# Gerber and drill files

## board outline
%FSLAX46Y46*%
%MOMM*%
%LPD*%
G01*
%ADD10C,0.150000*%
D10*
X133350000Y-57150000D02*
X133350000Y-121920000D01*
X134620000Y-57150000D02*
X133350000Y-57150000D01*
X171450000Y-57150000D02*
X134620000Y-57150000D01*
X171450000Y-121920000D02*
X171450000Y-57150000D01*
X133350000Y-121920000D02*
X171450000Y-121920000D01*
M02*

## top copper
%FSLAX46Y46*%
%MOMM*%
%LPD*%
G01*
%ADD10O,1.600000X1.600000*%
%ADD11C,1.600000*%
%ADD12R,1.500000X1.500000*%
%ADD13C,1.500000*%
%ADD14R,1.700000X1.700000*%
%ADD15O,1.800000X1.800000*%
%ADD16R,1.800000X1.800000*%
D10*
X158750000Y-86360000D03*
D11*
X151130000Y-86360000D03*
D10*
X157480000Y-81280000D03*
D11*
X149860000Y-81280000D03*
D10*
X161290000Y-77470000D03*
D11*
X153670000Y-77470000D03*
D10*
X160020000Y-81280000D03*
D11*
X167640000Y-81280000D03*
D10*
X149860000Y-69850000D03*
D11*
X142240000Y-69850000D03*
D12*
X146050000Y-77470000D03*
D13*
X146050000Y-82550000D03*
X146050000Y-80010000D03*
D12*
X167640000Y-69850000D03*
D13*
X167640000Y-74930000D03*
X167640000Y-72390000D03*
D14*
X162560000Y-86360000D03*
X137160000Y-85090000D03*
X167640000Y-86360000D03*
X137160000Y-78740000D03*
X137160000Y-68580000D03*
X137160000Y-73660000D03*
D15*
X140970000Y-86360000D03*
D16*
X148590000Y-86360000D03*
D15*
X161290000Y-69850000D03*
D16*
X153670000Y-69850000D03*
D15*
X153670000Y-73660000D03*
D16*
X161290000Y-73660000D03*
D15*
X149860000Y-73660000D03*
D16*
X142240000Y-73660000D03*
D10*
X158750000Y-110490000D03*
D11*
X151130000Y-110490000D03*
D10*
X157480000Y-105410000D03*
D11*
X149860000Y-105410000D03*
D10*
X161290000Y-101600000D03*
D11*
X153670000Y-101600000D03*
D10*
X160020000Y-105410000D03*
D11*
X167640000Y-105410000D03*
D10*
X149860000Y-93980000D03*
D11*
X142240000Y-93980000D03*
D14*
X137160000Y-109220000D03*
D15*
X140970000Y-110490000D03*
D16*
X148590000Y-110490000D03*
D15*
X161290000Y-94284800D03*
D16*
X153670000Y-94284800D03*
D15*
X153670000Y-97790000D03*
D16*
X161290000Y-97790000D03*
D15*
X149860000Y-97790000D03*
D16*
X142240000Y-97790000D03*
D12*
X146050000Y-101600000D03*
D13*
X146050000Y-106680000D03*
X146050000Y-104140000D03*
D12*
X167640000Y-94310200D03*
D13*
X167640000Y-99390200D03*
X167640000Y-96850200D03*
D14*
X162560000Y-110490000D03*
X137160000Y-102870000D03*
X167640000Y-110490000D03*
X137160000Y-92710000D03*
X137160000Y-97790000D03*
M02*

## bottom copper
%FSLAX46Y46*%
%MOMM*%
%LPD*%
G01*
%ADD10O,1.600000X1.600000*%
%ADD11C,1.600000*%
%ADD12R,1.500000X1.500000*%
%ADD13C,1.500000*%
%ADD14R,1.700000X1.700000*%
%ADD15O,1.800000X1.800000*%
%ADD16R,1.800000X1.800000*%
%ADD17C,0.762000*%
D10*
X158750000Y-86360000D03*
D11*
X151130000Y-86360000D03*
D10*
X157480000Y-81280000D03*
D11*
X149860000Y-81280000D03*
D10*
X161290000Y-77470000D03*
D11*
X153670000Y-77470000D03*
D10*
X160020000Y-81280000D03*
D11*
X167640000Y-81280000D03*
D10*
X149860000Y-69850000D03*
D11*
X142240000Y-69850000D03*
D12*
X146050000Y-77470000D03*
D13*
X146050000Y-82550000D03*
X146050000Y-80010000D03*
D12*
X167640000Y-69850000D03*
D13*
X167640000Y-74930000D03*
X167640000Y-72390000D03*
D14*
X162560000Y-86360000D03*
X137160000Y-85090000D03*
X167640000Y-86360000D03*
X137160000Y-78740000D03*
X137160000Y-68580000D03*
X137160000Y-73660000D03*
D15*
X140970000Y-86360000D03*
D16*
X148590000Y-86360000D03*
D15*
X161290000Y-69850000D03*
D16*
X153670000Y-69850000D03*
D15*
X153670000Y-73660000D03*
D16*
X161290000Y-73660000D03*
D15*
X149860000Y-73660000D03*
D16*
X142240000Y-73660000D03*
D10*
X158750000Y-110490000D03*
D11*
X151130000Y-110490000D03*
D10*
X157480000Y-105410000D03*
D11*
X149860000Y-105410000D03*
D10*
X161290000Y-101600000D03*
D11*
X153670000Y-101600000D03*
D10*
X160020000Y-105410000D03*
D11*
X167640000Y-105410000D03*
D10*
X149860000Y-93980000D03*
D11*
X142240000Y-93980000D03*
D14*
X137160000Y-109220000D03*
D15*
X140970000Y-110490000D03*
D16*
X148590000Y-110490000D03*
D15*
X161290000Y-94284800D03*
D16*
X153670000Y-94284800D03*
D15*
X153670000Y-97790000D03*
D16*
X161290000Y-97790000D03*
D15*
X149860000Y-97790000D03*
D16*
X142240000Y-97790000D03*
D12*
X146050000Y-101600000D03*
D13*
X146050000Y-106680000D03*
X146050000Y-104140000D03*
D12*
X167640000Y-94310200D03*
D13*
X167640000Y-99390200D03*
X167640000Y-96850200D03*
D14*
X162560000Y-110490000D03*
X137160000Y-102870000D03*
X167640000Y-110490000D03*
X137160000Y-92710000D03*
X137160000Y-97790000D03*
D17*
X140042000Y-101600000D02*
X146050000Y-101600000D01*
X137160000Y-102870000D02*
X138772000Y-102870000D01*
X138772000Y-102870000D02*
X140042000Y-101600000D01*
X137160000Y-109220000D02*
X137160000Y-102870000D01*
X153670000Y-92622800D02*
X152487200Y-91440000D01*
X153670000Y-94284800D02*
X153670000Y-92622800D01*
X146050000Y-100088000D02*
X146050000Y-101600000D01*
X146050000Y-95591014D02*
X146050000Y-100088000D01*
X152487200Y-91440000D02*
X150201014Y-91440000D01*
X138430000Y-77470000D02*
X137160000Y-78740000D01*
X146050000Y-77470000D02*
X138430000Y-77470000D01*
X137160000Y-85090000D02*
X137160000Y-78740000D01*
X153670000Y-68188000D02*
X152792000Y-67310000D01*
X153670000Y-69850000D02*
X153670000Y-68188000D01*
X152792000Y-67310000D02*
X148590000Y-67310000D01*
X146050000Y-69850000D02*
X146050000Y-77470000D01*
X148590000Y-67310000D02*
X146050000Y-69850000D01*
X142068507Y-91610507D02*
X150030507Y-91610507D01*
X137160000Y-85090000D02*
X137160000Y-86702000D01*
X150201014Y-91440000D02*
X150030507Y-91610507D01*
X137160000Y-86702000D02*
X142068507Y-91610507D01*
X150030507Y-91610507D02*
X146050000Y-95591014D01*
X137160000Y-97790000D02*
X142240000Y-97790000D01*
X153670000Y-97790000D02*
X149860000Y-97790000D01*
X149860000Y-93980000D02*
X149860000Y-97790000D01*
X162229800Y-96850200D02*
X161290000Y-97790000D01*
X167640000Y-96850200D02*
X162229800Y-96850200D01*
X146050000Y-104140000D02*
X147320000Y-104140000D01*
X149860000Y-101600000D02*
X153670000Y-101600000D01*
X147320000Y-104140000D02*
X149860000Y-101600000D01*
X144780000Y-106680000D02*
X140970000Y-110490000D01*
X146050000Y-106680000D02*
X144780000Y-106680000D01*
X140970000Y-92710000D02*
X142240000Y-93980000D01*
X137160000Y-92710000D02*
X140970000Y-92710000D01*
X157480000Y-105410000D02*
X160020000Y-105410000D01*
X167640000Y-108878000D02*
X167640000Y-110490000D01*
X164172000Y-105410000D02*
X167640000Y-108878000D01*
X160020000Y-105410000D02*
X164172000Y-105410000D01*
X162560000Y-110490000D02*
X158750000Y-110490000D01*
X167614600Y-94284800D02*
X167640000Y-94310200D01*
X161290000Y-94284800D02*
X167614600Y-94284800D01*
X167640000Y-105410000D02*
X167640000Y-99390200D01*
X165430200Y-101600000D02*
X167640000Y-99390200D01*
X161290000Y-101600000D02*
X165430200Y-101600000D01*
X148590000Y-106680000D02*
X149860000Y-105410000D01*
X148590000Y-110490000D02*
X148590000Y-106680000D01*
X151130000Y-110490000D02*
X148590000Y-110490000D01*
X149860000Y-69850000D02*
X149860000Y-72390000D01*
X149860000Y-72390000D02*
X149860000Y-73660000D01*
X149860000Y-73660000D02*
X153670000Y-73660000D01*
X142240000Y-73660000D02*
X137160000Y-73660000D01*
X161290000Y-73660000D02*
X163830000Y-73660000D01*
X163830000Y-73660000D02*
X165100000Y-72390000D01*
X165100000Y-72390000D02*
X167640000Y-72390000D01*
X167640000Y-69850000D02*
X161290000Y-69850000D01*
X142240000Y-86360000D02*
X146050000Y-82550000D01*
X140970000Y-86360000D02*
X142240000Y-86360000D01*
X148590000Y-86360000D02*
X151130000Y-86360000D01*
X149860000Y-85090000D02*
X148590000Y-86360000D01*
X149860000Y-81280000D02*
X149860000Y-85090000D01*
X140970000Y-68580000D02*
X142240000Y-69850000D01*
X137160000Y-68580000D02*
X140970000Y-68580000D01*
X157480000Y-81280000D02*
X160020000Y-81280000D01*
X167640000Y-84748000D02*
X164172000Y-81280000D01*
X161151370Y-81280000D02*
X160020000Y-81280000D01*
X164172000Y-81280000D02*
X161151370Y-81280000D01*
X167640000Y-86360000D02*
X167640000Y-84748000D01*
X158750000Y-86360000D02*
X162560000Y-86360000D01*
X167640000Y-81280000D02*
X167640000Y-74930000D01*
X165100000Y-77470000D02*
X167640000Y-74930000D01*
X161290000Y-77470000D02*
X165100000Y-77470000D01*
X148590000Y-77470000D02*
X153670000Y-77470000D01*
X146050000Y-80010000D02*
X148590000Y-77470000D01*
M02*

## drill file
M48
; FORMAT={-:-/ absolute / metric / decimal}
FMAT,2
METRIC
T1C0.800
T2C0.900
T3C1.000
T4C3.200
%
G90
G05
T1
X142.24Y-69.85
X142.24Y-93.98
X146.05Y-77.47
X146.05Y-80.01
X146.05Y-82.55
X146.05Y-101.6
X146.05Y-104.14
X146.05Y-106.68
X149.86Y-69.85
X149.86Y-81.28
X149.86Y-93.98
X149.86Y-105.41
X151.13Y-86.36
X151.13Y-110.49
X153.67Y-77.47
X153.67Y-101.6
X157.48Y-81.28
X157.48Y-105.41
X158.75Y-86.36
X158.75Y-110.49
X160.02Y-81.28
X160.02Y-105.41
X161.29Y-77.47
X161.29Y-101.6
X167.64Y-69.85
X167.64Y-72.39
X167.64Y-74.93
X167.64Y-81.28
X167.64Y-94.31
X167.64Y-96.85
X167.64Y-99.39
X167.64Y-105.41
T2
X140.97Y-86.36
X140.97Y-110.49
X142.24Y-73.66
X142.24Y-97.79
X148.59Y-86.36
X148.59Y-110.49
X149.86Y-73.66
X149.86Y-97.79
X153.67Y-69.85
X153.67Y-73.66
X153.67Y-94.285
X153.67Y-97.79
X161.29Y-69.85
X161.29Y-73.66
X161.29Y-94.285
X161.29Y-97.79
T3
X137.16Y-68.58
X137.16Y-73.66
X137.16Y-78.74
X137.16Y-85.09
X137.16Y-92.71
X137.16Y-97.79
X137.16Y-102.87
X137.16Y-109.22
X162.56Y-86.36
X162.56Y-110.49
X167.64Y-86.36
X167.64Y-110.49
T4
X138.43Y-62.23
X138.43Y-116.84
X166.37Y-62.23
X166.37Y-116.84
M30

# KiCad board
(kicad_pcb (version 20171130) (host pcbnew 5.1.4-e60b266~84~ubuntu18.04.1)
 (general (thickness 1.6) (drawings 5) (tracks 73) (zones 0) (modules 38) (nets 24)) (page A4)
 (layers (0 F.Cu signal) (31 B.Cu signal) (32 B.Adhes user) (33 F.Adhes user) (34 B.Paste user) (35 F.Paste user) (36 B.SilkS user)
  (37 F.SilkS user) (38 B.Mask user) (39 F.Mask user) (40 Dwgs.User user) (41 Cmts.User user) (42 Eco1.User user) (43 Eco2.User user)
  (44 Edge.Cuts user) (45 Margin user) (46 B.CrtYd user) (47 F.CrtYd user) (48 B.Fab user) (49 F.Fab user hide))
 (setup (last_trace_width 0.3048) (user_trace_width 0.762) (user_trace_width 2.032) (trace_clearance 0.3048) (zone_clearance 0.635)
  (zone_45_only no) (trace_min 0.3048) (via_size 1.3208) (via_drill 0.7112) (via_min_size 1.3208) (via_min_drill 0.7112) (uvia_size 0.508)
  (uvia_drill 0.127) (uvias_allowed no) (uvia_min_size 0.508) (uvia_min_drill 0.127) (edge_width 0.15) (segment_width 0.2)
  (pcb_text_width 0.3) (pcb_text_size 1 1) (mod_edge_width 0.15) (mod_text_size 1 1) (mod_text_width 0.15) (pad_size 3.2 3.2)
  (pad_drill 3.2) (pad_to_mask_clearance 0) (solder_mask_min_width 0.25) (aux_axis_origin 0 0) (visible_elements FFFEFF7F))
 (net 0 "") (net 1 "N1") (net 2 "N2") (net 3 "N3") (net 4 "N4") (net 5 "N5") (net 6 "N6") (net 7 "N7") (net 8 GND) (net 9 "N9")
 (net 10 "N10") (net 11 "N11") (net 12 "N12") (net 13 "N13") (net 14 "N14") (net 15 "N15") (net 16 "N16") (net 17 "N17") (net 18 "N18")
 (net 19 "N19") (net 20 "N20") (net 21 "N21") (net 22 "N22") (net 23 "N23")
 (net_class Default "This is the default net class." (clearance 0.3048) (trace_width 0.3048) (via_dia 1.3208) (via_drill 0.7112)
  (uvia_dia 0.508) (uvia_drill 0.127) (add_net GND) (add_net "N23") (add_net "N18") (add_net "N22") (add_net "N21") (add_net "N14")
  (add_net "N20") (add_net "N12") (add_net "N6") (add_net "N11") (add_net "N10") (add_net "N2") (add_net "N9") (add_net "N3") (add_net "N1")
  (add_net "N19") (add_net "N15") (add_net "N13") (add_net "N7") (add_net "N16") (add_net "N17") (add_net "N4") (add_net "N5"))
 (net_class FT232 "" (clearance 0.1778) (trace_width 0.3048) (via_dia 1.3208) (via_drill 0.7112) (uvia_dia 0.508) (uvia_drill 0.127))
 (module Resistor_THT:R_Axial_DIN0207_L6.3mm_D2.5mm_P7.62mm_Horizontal (layer F.Cu) (at 151.13 86.36)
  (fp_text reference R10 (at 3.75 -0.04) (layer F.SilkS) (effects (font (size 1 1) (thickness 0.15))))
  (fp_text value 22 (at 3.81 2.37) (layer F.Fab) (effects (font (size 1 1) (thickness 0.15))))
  (pad 2 thru_hole oval (at 7.62 0) (size 1.6 1.6) (drill 0.8) (layers *.Cu *.Mask) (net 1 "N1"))
  (pad 1 thru_hole circle (at 0 0) (size 1.6 1.6) (drill 0.8) (layers *.Cu *.Mask) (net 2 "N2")))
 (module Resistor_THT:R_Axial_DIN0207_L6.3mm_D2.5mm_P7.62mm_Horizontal (layer F.Cu) (at 149.86 81.28)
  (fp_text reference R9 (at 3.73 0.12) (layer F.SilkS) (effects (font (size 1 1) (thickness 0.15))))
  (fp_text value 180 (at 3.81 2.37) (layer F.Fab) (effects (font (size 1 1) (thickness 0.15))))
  (pad 2 thru_hole oval (at 7.62 0) (size 1.6 1.6) (drill 0.8) (layers *.Cu *.Mask) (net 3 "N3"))
  (pad 1 thru_hole circle (at 0 0) (size 1.6 1.6) (drill 0.8) (layers *.Cu *.Mask) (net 2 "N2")))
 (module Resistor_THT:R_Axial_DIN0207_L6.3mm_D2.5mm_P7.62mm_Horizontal (layer F.Cu) (at 153.67 77.47)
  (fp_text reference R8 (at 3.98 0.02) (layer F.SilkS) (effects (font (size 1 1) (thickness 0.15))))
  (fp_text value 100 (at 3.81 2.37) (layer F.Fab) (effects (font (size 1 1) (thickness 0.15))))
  (pad 2 thru_hole oval (at 7.62 0) (size 1.6 1.6) (drill 0.8) (layers *.Cu *.Mask) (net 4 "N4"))
  (pad 1 thru_hole circle (at 0 0) (size 1.6 1.6) (drill 0.8) (layers *.Cu *.Mask) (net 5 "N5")))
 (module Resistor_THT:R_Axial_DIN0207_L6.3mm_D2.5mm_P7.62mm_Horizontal (layer F.Cu) (at 167.64 81.28 180)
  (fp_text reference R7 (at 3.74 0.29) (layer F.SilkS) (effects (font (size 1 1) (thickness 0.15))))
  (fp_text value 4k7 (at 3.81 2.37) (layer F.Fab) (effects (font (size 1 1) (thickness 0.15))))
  (pad 2 thru_hole oval (at 7.62 0 180) (size 1.6 1.6) (drill 0.8) (layers *.Cu *.Mask) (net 3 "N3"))
  (pad 1 thru_hole circle (at 0 0 180) (size 1.6 1.6) (drill 0.8) (layers *.Cu *.Mask) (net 4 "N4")))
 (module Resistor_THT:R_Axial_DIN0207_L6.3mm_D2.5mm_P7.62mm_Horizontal (layer F.Cu) (at 142.24 69.85)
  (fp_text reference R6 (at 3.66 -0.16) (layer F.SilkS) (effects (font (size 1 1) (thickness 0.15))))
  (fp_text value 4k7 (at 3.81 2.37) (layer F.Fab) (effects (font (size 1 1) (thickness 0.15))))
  (pad 2 thru_hole oval (at 7.62 0) (size 1.6 1.6) (drill 0.8) (layers *.Cu *.Mask) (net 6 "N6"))
  (pad 1 thru_hole circle (at 0 0) (size 1.6 1.6) (drill 0.8) (layers *.Cu *.Mask) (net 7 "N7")))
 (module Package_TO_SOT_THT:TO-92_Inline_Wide (layer F.Cu) (at 146.05 77.47 270)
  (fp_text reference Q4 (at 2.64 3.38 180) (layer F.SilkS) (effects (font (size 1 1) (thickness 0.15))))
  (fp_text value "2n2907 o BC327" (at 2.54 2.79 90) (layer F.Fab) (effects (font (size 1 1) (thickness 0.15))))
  (pad 1 thru_hole rect (at 0 0) (size 1.5 1.5) (drill 0.8) (layers *.Cu *.Mask) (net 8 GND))
  (pad 3 thru_hole circle (at 5.08 0) (size 1.5 1.5) (drill 0.8) (layers *.Cu *.Mask) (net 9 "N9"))
  (pad 2 thru_hole circle (at 2.54 0) (size 1.5 1.5) (drill 0.8) (layers *.Cu *.Mask) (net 5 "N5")))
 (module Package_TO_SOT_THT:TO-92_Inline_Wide (layer F.Cu) (at 167.64 69.85 270)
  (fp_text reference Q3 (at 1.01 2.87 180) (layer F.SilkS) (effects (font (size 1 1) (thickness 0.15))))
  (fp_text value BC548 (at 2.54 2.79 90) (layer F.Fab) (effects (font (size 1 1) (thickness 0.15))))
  (pad 1 thru_hole rect (at 0 0) (size 1.5 1.5) (drill 0.8) (layers *.Cu *.Mask) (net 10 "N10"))
  (pad 3 thru_hole circle (at 5.08 0) (size 1.5 1.5) (drill 0.8) (layers *.Cu *.Mask) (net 4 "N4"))
  (pad 2 thru_hole circle (at 2.54 0) (size 1.5 1.5) (drill 0.8) (layers *.Cu *.Mask) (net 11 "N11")))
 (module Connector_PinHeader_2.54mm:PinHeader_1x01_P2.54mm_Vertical (layer F.Cu) (at 162.56 86.36)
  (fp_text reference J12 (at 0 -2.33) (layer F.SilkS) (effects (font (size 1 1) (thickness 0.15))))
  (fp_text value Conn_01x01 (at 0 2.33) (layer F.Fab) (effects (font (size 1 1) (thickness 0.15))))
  (pad 1 thru_hole rect (at 0 0) (size 1.7 1.7) (drill 1) (layers *.Cu *.Mask) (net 1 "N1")))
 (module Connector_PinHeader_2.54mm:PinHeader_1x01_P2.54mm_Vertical (layer F.Cu) (at 137.16 85.09)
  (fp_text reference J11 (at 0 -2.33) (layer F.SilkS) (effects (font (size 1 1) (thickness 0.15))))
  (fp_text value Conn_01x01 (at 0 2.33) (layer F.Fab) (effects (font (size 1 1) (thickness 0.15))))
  (pad 1 thru_hole rect (at 0 0) (size 1.7 1.7) (drill 1) (layers *.Cu *.Mask) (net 8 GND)))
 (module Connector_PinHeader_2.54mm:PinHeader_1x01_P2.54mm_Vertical (layer F.Cu) (at 167.64 86.36)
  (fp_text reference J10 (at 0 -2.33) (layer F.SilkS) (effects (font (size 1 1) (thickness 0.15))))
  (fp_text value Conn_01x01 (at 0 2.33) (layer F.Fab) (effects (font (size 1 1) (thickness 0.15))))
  (pad 1 thru_hole rect (at 0 0) (size 1.7 1.7) (drill 1) (layers *.Cu *.Mask) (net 3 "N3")))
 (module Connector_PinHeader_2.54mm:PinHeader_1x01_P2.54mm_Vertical (layer F.Cu) (at 137.16 78.74)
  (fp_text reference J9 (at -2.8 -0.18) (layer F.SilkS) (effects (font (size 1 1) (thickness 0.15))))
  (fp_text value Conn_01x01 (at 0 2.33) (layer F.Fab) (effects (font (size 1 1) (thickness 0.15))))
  (pad 1 thru_hole rect (at 0 0) (size 1.7 1.7) (drill 1) (layers *.Cu *.Mask) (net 8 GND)))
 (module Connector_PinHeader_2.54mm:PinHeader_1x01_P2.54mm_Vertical (layer F.Cu) (at 137.16 68.58)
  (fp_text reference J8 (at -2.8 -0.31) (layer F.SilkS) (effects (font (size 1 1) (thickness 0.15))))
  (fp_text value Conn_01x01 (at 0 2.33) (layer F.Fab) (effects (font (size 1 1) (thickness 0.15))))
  (pad 1 thru_hole rect (at 0 0) (size 1.7 1.7) (drill 1) (layers *.Cu *.Mask) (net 7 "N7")))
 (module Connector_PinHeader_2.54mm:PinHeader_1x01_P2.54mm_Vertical (layer F.Cu) (at 137.16 73.66)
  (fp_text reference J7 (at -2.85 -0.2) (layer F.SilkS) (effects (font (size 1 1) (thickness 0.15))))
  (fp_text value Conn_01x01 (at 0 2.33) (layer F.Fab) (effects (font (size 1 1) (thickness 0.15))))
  (pad 1 thru_hole rect (at 0 0) (size 1.7 1.7) (drill 1) (layers *.Cu *.Mask) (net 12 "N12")))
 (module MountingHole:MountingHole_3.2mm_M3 (layer F.Cu) (at 138.43 62.23)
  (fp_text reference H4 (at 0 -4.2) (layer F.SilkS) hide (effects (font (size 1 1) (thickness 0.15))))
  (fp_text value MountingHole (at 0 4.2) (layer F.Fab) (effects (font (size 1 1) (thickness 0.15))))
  (pad 1 np_thru_hole circle (at 0 0) (size 3.2 3.2) (drill 3.2) (layers *.Cu *.Mask)))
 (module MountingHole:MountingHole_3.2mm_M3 (layer F.Cu) (at 166.37 116.84)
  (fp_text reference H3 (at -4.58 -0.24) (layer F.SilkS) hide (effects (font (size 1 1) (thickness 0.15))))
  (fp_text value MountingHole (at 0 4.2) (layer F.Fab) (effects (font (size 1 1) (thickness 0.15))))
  (pad 1 np_thru_hole circle (at 0 0) (size 3.2 3.2) (drill 3.2) (layers *.Cu *.Mask)))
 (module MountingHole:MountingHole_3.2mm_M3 (layer F.Cu) (at 138.43 116.84)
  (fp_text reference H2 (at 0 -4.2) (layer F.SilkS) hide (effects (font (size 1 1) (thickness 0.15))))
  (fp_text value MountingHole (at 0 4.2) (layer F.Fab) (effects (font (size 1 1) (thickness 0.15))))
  (pad 1 np_thru_hole circle (at 0 0) (size 3.2 3.2) (drill 3.2) (layers *.Cu *.Mask)))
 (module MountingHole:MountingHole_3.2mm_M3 (layer F.Cu) (at 166.37 62.23)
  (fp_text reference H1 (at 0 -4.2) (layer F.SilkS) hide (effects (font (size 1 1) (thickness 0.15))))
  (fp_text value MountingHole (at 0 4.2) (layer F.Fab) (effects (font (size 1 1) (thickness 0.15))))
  (pad 1 np_thru_hole circle (at 0 0) (size 3.2 3.2) (drill 3.2) (layers *.Cu *.Mask)))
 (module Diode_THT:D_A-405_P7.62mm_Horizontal (layer F.Cu) (at 148.59 86.36 180)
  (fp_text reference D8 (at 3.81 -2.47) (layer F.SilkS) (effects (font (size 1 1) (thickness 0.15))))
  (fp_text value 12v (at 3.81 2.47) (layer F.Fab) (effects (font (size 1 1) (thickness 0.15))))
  (pad 2 thru_hole oval (at 7.62 0 180) (size 1.8 1.8) (drill 0.9) (layers *.Cu *.Mask) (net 9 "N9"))
  (pad 1 thru_hole rect (at 0 0 180) (size 1.8 1.8) (drill 0.9) (layers *.Cu *.Mask) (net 2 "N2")))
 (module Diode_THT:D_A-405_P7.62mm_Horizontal (layer F.Cu) (at 153.67 69.85)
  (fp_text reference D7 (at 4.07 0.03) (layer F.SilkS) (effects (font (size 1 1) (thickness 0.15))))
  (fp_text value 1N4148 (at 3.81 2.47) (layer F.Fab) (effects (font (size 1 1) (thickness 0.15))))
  (pad 2 thru_hole oval (at 7.62 0) (size 1.8 1.8) (drill 0.9) (layers *.Cu *.Mask) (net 10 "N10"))
  (pad 1 thru_hole rect (at 0 0) (size 1.8 1.8) (drill 0.9) (layers *.Cu *.Mask) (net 8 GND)))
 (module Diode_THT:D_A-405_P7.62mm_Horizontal (layer F.Cu) (at 161.29 73.66 180)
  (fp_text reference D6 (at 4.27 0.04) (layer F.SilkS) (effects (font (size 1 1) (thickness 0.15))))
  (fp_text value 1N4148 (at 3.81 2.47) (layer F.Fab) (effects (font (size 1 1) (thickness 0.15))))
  (pad 2 thru_hole oval (at 7.62 0 180) (size 1.8 1.8) (drill 0.9) (layers *.Cu *.Mask) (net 6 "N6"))
  (pad 1 thru_hole rect (at 0 0 180) (size 1.8 1.8) (drill 0.9) (layers *.Cu *.Mask) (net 11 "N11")))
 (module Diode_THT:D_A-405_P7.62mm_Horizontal (layer F.Cu) (at 142.24 73.66)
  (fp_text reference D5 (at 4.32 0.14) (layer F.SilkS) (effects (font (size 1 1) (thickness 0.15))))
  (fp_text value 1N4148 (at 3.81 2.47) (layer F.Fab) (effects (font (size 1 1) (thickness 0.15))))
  (pad 2 thru_hole oval (at 7.62 0) (size 1.8 1.8) (drill 0.9) (layers *.Cu *.Mask) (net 6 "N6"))
  (pad 1 thru_hole rect (at 0 0) (size 1.8 1.8) (drill 0.9) (layers *.Cu *.Mask) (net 12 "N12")))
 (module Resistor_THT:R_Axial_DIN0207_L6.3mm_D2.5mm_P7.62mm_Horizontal (layer F.Cu) (at 151.13 110.49)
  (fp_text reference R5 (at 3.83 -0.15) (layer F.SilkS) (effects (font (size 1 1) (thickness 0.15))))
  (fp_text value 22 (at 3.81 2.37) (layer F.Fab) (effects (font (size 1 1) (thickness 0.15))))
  (pad 2 thru_hole oval (at 7.62 0) (size 1.6 1.6) (drill 0.8) (layers *.Cu *.Mask) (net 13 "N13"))
  (pad 1 thru_hole circle (at 0 0) (size 1.6 1.6) (drill 0.8) (layers *.Cu *.Mask) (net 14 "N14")))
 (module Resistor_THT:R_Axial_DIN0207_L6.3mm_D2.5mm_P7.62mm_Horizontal (layer F.Cu) (at 149.86 105.41)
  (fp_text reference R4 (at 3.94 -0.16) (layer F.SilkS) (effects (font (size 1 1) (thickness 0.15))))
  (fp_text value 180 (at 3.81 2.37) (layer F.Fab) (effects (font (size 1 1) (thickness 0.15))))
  (pad 2 thru_hole oval (at 7.62 0) (size 1.6 1.6) (drill 0.8) (layers *.Cu *.Mask) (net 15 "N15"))
  (pad 1 thru_hole circle (at 0 0) (size 1.6 1.6) (drill 0.8) (layers *.Cu *.Mask) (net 14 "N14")))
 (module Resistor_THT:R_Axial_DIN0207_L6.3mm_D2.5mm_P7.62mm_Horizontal (layer F.Cu) (at 153.67 101.6)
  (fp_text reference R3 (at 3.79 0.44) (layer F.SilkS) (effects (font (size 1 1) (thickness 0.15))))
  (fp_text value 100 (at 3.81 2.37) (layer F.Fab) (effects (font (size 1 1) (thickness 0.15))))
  (pad 2 thru_hole oval (at 7.62 0) (size 1.6 1.6) (drill 0.8) (layers *.Cu *.Mask) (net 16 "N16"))
  (pad 1 thru_hole circle (at 0 0) (size 1.6 1.6) (drill 0.8) (layers *.Cu *.Mask) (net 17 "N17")))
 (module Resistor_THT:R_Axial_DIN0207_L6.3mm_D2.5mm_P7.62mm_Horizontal (layer F.Cu) (at 167.64 105.41 180)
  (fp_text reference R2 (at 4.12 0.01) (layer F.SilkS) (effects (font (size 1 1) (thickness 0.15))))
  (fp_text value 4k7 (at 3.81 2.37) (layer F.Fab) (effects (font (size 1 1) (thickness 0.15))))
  (pad 2 thru_hole oval (at 7.62 0 180) (size 1.6 1.6) (drill 0.8) (layers *.Cu *.Mask) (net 15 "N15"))
  (pad 1 thru_hole circle (at 0 0 180) (size 1.6 1.6) (drill 0.8) (layers *.Cu *.Mask) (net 16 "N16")))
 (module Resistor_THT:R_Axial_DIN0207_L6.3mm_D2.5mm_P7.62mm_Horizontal (layer F.Cu) (at 142.24 93.98)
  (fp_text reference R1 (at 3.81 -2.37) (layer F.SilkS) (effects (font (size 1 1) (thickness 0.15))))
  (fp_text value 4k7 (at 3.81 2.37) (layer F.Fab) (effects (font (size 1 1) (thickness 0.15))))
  (pad 2 thru_hole oval (at 7.62 0) (size 1.6 1.6) (drill 0.8) (layers *.Cu *.Mask) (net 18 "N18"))
  (pad 1 thru_hole circle (at 0 0) (size 1.6 1.6) (drill 0.8) (layers *.Cu *.Mask) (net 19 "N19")))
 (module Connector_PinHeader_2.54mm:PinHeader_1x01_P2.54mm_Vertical (layer F.Cu) (at 137.16 109.22)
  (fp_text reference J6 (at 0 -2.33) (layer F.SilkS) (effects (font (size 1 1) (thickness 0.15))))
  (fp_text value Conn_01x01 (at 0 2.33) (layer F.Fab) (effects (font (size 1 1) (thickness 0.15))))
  (pad 1 thru_hole rect (at 0 0) (size 1.7 1.7) (drill 1) (layers *.Cu *.Mask) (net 8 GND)))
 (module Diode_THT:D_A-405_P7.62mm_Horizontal (layer F.Cu) (at 148.59 110.49 180)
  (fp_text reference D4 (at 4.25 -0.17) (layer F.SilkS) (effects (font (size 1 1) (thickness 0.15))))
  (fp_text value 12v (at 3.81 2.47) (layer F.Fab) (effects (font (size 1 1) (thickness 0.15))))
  (pad 2 thru_hole oval (at 7.62 0 180) (size 1.8 1.8) (drill 0.9) (layers *.Cu *.Mask) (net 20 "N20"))
  (pad 1 thru_hole rect (at 0 0 180) (size 1.8 1.8) (drill 0.9) (layers *.Cu *.Mask) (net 14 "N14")))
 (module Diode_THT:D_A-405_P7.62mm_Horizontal (layer F.Cu) (at 153.67 94.2848)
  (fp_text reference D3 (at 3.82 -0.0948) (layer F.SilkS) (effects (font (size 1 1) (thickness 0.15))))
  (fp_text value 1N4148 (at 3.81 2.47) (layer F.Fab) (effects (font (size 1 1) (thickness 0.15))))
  (pad 2 thru_hole oval (at 7.62 0) (size 1.8 1.8) (drill 0.9) (layers *.Cu *.Mask) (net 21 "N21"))
  (pad 1 thru_hole rect (at 0 0) (size 1.8 1.8) (drill 0.9) (layers *.Cu *.Mask) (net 8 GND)))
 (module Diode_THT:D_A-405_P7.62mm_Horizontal (layer F.Cu) (at 161.29 97.79 180)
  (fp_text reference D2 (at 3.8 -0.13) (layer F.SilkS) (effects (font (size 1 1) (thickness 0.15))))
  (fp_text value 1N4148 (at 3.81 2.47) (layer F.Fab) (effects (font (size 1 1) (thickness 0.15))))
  (pad 2 thru_hole oval (at 7.62 0 180) (size 1.8 1.8) (drill 0.9) (layers *.Cu *.Mask) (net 18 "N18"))
  (pad 1 thru_hole rect (at 0 0 180) (size 1.8 1.8) (drill 0.9) (layers *.Cu *.Mask) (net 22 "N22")))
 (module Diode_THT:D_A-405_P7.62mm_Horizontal (layer F.Cu) (at 142.24 97.79)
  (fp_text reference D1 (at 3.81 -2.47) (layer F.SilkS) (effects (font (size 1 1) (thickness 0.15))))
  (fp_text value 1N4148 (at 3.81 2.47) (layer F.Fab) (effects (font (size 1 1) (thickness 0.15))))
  (pad 2 thru_hole oval (at 7.62 0) (size 1.8 1.8) (drill 0.9) (layers *.Cu *.Mask) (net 18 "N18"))
  (pad 1 thru_hole rect (at 0 0) (size 1.8 1.8) (drill 0.9) (layers *.Cu *.Mask) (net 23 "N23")))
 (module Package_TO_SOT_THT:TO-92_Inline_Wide (layer F.Cu) (at 146.05 101.6 270)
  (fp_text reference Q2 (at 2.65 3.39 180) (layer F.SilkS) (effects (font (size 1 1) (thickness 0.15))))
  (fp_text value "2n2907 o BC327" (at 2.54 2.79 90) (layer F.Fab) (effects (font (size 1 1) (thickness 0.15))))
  (pad 1 thru_hole rect (at 0 0) (size 1.5 1.5) (drill 0.8) (layers *.Cu *.Mask) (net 8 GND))
  (pad 3 thru_hole circle (at 5.08 0) (size 1.5 1.5) (drill 0.8) (layers *.Cu *.Mask) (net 20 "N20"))
  (pad 2 thru_hole circle (at 2.54 0) (size 1.5 1.5) (drill 0.8) (layers *.Cu *.Mask) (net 17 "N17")))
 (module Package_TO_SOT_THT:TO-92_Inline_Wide (layer F.Cu) (at 167.64 94.3102 270)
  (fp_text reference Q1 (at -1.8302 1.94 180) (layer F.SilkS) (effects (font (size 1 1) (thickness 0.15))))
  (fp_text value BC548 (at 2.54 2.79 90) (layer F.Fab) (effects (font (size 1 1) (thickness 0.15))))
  (pad 1 thru_hole rect (at 0 0) (size 1.5 1.5) (drill 0.8) (layers *.Cu *.Mask) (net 21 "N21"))
  (pad 3 thru_hole circle (at 5.08 0) (size 1.5 1.5) (drill 0.8) (layers *.Cu *.Mask) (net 16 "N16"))
  (pad 2 thru_hole circle (at 2.54 0) (size 1.5 1.5) (drill 0.8) (layers *.Cu *.Mask) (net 22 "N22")))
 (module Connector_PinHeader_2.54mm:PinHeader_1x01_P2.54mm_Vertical (layer F.Cu) (at 162.56 110.49)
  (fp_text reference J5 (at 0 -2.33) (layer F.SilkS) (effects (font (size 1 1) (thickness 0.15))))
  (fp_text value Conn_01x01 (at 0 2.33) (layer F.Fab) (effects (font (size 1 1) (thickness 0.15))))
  (pad 1 thru_hole rect (at 0 0) (size 1.7 1.7) (drill 1) (layers *.Cu *.Mask) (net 13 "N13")))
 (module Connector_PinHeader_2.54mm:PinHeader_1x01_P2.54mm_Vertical (layer F.Cu) (at 137.16 102.87)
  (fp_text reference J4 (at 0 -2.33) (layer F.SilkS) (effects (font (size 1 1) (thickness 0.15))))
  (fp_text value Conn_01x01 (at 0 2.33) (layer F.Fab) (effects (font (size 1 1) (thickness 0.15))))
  (pad 1 thru_hole rect (at 0 0) (size 1.7 1.7) (drill 1) (layers *.Cu *.Mask) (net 8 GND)))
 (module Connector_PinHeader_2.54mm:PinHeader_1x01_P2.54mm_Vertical (layer F.Cu) (at 167.64 110.49)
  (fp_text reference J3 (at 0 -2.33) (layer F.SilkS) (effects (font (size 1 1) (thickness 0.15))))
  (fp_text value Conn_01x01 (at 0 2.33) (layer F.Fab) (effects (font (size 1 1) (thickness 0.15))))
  (pad 1 thru_hole rect (at 0 0) (size 1.7 1.7) (drill 1) (layers *.Cu *.Mask) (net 15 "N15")))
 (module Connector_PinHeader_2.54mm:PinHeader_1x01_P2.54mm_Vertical (layer F.Cu) (at 137.16 92.71)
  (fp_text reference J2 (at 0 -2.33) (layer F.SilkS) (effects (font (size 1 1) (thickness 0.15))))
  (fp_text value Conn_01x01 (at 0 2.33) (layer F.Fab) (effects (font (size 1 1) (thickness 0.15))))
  (pad 1 thru_hole rect (at 0 0) (size 1.7 1.7) (drill 1) (layers *.Cu *.Mask) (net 19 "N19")))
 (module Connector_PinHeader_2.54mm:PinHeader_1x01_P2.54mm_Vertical (layer F.Cu) (at 137.16 97.79)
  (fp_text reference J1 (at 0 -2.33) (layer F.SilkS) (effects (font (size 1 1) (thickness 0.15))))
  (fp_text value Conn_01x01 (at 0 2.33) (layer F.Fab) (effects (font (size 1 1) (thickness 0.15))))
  (pad 1 thru_hole rect (at 0 0) (size 1.7 1.7) (drill 1) (layers *.Cu *.Mask) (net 23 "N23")))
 (gr_line (start 133.35 57.15) (end 133.35 121.92) (layer Edge.Cuts) (width 0.15))
 (gr_line (start 134.62 57.15) (end 133.35 57.15) (layer Edge.Cuts) (width 0.15))
 (gr_line (start 171.45 57.15) (end 134.62 57.15) (layer Edge.Cuts) (width 0.15))
 (gr_line (start 171.45 121.92) (end 171.45 57.15) (layer Edge.Cuts) (width 0.15))
 (gr_line (start 133.35 121.92) (end 171.45 121.92) (layer Edge.Cuts) (width 0.15))
 (segment (start 140.042 101.6) (end 146.05 101.6) (width 0.762) (layer B.Cu) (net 8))
 (segment (start 137.16 102.87) (end 138.772 102.87) (width 0.762) (layer B.Cu) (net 8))
 (segment (start 138.772 102.87) (end 140.042 101.6) (width 0.762) (layer B.Cu) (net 8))
 (segment (start 137.16 109.22) (end 137.16 102.87) (width 0.762) (layer B.Cu) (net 8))
 (segment (start 153.67 92.6228) (end 152.4872 91.44) (width 0.762) (layer B.Cu) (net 8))
 (segment (start 153.67 94.2848) (end 153.67 92.6228) (width 0.762) (layer B.Cu) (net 8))
 (segment (start 146.05 100.088) (end 146.05 101.6) (width 0.762) (layer B.Cu) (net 8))
 (segment (start 146.05 95.591014) (end 146.05 100.088) (width 0.762) (layer B.Cu) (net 8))
 (segment (start 152.4872 91.44) (end 150.201014 91.44) (width 0.762) (layer B.Cu) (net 8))
 (segment (start 138.43 77.47) (end 137.16 78.74) (width 0.762) (layer B.Cu) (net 8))
 (segment (start 146.05 77.47) (end 138.43 77.47) (width 0.762) (layer B.Cu) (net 8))
 (segment (start 137.16 85.09) (end 137.16 78.74) (width 0.762) (layer B.Cu) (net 8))
 (segment (start 153.67 68.188) (end 152.792 67.31) (width 0.762) (layer B.Cu) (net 8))
 (segment (start 153.67 69.85) (end 153.67 68.188) (width 0.762) (layer B.Cu) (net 8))
 (segment (start 152.792 67.31) (end 148.59 67.31) (width 0.762) (layer B.Cu) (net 8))
 (segment (start 146.05 69.85) (end 146.05 77.47) (width 0.762) (layer B.Cu) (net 8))
 (segment (start 148.59 67.31) (end 146.05 69.85) (width 0.762) (layer B.Cu) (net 8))
 (segment (start 142.068507 91.610507) (end 150.030507 91.610507) (width 0.762) (layer B.Cu) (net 8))
 (segment (start 137.16 85.09) (end 137.16 86.702) (width 0.762) (layer B.Cu) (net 8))
 (segment (start 150.201014 91.44) (end 150.030507 91.610507) (width 0.762) (layer B.Cu) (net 8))
 (segment (start 137.16 86.702) (end 142.068507 91.610507) (width 0.762) (layer B.Cu) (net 8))
 (segment (start 150.030507 91.610507) (end 146.05 95.591014) (width 0.762) (layer B.Cu) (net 8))
 (segment (start 137.16 97.79) (end 142.24 97.79) (width 0.762) (layer B.Cu) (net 23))
 (segment (start 153.67 97.79) (end 149.86 97.79) (width 0.762) (layer B.Cu) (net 18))
 (segment (start 149.86 93.98) (end 149.86 97.79) (width 0.762) (layer B.Cu) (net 18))
 (segment (start 162.2298 96.8502) (end 161.29 97.79) (width 0.762) (layer B.Cu) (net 22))
 (segment (start 167.64 96.8502) (end 162.2298 96.8502) (width 0.762) (layer B.Cu) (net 22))
 (segment (start 146.05 104.14) (end 147.32 104.14) (width 0.762) (layer B.Cu) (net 17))
 (segment (start 149.86 101.6) (end 153.67 101.6) (width 0.762) (layer B.Cu) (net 17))
 (segment (start 147.32 104.14) (end 149.86 101.6) (width 0.762) (layer B.Cu) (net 17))
 (segment (start 144.78 106.68) (end 140.97 110.49) (width 0.762) (layer B.Cu) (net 20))
 (segment (start 146.05 106.68) (end 144.78 106.68) (width 0.762) (layer B.Cu) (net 20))
 (segment (start 140.97 92.71) (end 142.24 93.98) (width 0.762) (layer B.Cu) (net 19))
 (segment (start 137.16 92.71) (end 140.97 92.71) (width 0.762) (layer B.Cu) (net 19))
 (segment (start 157.48 105.41) (end 160.02 105.41) (width 0.762) (layer B.Cu) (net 15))
 (segment (start 167.64 108.878) (end 167.64 110.49) (width 0.762) (layer B.Cu) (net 15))
 (segment (start 164.172 105.41) (end 167.64 108.878) (width 0.762) (layer B.Cu) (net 15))
 (segment (start 160.02 105.41) (end 164.172 105.41) (width 0.762) (layer B.Cu) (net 15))
 (segment (start 162.56 110.49) (end 158.75 110.49) (width 0.762) (layer B.Cu) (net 13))
 (segment (start 167.6146 94.2848) (end 167.64 94.3102) (width 0.762) (layer B.Cu) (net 21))
 (segment (start 161.29 94.2848) (end 167.6146 94.2848) (width 0.762) (layer B.Cu) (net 21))
 (segment (start 167.64 105.41) (end 167.64 99.3902) (width 0.762) (layer B.Cu) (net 16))
 (segment (start 165.4302 101.6) (end 167.64 99.3902) (width 0.762) (layer B.Cu) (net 16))
 (segment (start 161.29 101.6) (end 165.4302 101.6) (width 0.762) (layer B.Cu) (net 16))
 (segment (start 148.59 106.68) (end 149.86 105.41) (width 0.762) (layer B.Cu) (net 14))
 (segment (start 148.59 110.49) (end 148.59 106.68) (width 0.762) (layer B.Cu) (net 14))
 (segment (start 151.13 110.49) (end 148.59 110.49) (width 0.762) (layer B.Cu) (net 14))
 (segment (start 149.86 69.85) (end 149.86 72.39) (width 0.762) (layer B.Cu) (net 6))
 (segment (start 149.86 72.39) (end 149.86 73.66) (width 0.762) (layer B.Cu) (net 6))
 (segment (start 149.86 73.66) (end 153.67 73.66) (width 0.762) (layer B.Cu) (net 6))
 (segment (start 142.24 73.66) (end 137.16 73.66) (width 0.762) (layer B.Cu) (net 12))
 (segment (start 161.29 73.66) (end 163.83 73.66) (width 0.762) (layer B.Cu) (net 11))
 (segment (start 163.83 73.66) (end 165.1 72.39) (width 0.762) (layer B.Cu) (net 11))
 (segment (start 165.1 72.39) (end 167.64 72.39) (width 0.762) (layer B.Cu) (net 11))
 (segment (start 167.64 69.85) (end 161.29 69.85) (width 0.762) (layer B.Cu) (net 10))
 (segment (start 142.24 86.36) (end 146.05 82.55) (width 0.762) (layer B.Cu) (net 9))
 (segment (start 140.97 86.36) (end 142.24 86.36) (width 0.762) (layer B.Cu) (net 9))
 (segment (start 148.59 86.36) (end 151.13 86.36) (width 0.762) (layer B.Cu) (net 2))
 (segment (start 149.86 85.09) (end 148.59 86.36) (width 0.762) (layer B.Cu) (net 2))
 (segment (start 149.86 81.28) (end 149.86 85.09) (width 0.762) (layer B.Cu) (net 2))
 (segment (start 140.97 68.58) (end 142.24 69.85) (width 0.762) (layer B.Cu) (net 7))
 (segment (start 137.16 68.58) (end 140.97 68.58) (width 0.762) (layer B.Cu) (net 7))
 (segment (start 157.48 81.28) (end 160.02 81.28) (width 0.762) (layer B.Cu) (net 3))
 (segment (start 167.64 84.748) (end 164.172 81.28) (width 0.762) (layer B.Cu) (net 3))
 (segment (start 161.15137 81.28) (end 160.02 81.28) (width 0.762) (layer B.Cu) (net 3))
 (segment (start 164.172 81.28) (end 161.15137 81.28) (width 0.762) (layer B.Cu) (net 3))
 (segment (start 167.64 86.36) (end 167.64 84.748) (width 0.762) (layer B.Cu) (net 3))
 (segment (start 158.75 86.36) (end 162.56 86.36) (width 0.762) (layer B.Cu) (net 1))
 (segment (start 167.64 81.28) (end 167.64 74.93) (width 0.762) (layer B.Cu) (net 4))
 (segment (start 165.1 77.47) (end 167.64 74.93) (width 0.762) (layer B.Cu) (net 4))
 (segment (start 161.29 77.47) (end 165.1 77.47) (width 0.762) (layer B.Cu) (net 4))
 (segment (start 148.59 77.47) (end 153.67 77.47) (width 0.762) (layer B.Cu) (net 5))
 (segment (start 146.05 80.01) (end 148.59 77.47) (width 0.762) (layer B.Cu) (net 5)))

